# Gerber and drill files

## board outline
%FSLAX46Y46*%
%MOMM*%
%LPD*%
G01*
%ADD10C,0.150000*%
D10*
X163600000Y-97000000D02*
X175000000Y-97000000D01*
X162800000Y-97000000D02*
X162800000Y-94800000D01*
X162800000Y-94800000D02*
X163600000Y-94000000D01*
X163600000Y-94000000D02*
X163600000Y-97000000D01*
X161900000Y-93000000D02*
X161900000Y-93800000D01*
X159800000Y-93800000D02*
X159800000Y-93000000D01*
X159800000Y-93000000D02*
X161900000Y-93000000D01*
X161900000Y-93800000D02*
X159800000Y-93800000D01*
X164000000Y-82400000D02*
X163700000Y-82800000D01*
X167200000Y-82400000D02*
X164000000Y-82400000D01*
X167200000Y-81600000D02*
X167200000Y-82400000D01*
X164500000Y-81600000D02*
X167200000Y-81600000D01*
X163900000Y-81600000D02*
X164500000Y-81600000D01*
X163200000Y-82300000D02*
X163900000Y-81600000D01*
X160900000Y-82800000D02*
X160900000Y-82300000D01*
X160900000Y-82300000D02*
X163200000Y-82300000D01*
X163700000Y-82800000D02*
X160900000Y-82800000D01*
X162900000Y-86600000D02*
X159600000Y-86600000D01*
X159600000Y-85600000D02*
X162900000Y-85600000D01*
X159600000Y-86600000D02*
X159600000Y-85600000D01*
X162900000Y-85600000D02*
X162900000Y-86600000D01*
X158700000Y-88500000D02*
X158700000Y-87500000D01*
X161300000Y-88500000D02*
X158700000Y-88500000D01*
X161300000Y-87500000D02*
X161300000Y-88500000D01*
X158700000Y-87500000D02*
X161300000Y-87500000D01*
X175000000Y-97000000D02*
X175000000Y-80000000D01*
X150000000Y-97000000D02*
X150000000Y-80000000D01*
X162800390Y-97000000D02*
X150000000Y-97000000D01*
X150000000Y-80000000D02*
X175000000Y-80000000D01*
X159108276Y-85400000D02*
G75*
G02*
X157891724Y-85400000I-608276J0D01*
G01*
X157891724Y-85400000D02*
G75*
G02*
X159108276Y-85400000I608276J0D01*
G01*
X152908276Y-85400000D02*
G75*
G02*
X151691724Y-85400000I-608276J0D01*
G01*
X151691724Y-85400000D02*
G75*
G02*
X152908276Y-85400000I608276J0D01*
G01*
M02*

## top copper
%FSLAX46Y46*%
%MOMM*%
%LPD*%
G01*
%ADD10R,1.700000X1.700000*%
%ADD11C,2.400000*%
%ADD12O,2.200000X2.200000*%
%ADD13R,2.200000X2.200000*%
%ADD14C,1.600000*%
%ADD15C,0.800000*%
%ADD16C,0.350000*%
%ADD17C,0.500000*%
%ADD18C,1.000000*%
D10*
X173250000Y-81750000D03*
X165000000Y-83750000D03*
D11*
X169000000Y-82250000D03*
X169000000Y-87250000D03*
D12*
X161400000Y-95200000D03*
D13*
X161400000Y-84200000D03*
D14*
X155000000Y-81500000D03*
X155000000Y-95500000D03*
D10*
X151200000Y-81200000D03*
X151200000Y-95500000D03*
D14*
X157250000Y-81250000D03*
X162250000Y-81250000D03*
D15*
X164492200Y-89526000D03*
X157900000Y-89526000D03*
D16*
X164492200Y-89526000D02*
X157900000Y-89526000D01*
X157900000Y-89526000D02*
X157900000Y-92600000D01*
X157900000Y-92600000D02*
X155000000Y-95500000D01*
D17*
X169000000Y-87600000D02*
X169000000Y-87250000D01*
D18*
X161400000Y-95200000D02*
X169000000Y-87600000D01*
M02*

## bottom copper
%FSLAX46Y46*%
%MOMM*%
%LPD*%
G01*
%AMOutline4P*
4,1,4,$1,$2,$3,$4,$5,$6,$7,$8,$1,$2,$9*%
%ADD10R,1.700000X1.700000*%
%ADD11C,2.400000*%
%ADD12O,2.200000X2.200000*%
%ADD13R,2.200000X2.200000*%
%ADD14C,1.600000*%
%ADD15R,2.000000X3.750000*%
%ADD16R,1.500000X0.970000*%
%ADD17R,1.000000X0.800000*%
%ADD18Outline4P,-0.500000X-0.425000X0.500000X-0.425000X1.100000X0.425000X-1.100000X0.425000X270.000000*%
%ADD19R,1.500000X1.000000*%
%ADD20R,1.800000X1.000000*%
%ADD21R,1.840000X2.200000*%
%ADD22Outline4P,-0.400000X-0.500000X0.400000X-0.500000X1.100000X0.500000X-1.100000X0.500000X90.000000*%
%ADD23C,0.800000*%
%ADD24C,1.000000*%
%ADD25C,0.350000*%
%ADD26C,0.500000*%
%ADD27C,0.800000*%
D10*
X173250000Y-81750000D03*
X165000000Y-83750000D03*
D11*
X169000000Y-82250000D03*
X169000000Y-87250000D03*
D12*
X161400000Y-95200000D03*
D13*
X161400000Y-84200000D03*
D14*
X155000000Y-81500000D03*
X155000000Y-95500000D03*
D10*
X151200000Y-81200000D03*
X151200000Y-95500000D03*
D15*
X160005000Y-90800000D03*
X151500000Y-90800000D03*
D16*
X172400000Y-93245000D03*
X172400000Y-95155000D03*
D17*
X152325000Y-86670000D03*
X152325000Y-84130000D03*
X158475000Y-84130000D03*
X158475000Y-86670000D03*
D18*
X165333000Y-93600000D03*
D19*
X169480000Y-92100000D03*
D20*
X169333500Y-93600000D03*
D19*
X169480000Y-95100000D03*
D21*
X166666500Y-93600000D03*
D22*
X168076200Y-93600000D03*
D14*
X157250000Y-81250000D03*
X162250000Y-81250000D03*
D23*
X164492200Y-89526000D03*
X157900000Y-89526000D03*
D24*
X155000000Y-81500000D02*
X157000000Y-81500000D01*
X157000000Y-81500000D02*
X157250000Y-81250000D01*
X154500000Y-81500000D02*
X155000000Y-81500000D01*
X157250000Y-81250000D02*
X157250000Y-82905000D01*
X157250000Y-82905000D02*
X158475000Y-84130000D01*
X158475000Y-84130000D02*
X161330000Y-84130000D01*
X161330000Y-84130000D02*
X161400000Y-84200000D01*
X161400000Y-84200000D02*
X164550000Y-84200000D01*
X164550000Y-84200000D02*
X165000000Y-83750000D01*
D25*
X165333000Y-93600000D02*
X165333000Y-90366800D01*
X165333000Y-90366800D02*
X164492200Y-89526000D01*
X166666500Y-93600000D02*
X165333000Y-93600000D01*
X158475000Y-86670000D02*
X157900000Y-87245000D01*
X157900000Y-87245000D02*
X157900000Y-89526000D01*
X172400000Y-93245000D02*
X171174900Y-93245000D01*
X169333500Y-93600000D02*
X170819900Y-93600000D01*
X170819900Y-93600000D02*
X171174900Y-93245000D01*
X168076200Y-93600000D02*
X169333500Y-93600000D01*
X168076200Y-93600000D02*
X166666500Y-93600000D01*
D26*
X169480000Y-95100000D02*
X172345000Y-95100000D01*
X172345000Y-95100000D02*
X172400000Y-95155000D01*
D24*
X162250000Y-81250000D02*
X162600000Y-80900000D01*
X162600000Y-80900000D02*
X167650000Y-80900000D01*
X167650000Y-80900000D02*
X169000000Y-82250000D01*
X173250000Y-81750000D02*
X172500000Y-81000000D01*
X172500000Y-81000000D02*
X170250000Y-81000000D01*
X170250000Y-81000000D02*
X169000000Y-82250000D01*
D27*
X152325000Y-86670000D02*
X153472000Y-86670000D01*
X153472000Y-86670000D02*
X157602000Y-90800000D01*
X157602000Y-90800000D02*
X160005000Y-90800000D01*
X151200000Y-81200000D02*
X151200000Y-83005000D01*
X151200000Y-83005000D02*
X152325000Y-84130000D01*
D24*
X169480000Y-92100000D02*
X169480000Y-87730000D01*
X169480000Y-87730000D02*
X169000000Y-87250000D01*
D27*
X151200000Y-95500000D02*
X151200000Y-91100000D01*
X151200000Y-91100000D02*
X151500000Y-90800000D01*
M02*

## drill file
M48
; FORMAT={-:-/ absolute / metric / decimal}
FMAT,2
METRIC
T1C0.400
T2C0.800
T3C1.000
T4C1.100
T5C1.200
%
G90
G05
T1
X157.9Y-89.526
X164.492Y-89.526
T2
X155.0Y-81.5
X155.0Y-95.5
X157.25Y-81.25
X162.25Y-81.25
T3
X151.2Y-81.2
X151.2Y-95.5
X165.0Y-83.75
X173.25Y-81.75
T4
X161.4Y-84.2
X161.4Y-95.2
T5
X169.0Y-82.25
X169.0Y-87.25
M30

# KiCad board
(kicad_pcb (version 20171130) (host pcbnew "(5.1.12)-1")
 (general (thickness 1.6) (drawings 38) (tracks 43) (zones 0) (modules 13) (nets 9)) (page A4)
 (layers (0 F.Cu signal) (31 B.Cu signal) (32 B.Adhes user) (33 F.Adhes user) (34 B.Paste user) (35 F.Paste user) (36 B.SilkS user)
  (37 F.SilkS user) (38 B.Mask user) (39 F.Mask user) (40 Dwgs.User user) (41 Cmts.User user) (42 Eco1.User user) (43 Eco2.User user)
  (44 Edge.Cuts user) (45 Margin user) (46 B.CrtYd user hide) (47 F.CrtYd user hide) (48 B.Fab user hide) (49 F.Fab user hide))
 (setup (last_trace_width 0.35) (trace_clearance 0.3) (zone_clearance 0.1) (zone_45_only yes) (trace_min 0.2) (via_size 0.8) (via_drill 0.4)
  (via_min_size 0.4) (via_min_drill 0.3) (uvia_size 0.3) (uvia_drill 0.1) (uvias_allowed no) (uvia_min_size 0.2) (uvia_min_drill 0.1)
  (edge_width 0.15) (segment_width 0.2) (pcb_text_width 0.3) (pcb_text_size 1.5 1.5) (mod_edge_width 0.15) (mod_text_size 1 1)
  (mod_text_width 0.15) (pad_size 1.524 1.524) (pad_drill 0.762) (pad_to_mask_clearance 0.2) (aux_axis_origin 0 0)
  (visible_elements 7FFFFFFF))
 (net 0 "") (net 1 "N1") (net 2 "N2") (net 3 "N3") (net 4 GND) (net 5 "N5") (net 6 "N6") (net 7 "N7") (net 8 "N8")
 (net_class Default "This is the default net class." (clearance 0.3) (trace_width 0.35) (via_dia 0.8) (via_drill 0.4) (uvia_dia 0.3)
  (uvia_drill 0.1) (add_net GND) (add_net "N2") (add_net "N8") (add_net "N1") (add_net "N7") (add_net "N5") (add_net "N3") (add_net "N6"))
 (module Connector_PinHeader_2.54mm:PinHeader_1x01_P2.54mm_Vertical (layer F.Cu) (at 173.25 81.75)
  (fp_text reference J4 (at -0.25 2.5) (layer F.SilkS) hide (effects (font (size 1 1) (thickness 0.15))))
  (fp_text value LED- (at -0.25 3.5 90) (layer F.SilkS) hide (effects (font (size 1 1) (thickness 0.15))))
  (pad 1 thru_hole rect (at 0 0) (size 1.7 1.7) (drill 1) (layers *.Cu *.Mask) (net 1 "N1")))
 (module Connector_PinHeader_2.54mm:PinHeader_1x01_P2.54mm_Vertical (layer F.Cu) (at 165 83.75)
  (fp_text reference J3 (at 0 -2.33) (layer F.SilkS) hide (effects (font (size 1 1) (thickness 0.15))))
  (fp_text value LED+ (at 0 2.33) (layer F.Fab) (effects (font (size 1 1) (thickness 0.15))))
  (pad 1 thru_hole rect (at 0 0) (size 1.7 1.7) (drill 1) (layers *.Cu *.Mask) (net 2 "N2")))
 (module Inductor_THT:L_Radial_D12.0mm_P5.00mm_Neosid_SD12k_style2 (layer F.Cu) (at 169 82.25 270)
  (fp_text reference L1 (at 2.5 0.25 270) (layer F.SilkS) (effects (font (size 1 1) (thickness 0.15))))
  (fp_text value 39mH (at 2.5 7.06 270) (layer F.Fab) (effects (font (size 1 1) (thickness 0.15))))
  (pad 1 thru_hole circle (at 0 0 270) (size 2.4 2.4) (drill 1.2) (layers *.Cu *.Mask) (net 1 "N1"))
  (pad 2 thru_hole circle (at 5 0 270) (size 2.4 2.4) (drill 1.2) (layers *.Cu *.Mask) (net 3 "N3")))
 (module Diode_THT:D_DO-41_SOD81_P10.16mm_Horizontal (layer F.Cu) (at 161.4 84.2 270)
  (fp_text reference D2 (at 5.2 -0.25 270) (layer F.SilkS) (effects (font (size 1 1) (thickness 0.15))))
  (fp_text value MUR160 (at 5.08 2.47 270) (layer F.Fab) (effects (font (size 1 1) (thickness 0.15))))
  (pad 2 thru_hole oval (at 11 0 270) (size 2.2 2.2) (drill 1.1) (layers *.Cu *.Mask) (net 3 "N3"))
  (pad 1 thru_hole rect (at 0 0 270) (size 2.2 2.2) (drill 1.1) (layers *.Cu *.Mask) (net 2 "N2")))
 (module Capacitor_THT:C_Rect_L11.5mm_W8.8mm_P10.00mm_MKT (layer F.Cu) (at 155 83.5 270)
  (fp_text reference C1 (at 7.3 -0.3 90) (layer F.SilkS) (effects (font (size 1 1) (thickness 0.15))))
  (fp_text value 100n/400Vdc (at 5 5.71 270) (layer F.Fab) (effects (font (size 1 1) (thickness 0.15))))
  (pad 1 thru_hole circle (at -2 0 270) (size 1.6 1.6) (drill 0.8) (layers *.Cu *.Mask) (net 2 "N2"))
  (pad 2 thru_hole circle (at 12 0 270) (size 1.6 1.6) (drill 0.8) (layers *.Cu *.Mask) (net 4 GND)))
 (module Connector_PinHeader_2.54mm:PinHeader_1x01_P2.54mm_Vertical (layer F.Cu) (at 151.2 81.2)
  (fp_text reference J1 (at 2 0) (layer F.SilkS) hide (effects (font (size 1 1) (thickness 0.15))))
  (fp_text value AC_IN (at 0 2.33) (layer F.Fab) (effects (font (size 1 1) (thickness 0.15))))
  (pad 1 thru_hole rect (at 0 0) (size 1.7 1.7) (drill 1) (layers *.Cu *.Mask) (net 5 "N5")))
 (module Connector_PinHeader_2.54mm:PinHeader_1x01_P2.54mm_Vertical (layer F.Cu) (at 151.2 95.5)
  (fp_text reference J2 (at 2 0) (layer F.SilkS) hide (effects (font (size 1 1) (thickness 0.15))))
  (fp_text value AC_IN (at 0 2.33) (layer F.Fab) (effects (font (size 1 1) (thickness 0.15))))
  (pad 1 thru_hole rect (at 0 0) (size 1.7 1.7) (drill 1) (layers *.Cu *.Mask) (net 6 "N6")))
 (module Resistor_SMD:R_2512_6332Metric (layer B.Cu) (at 157 90.8 180)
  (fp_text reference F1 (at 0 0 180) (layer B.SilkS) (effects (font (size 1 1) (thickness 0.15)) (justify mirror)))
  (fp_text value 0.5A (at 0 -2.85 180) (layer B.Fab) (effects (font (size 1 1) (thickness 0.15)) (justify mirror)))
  (pad 1 smd rect (at -3.005 0 180) (size 2 3.75) (layers B.Cu B.Paste B.Mask) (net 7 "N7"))
  (pad 2 smd rect (at 5.5 0 180) (size 2 3.75) (layers B.Cu B.Paste B.Mask) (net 6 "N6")))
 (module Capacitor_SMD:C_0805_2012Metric (layer B.Cu) (at 172.4 94.2 270)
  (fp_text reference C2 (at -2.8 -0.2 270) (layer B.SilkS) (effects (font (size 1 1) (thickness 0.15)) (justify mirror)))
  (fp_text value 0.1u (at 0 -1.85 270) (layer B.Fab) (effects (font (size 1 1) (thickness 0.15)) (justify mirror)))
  (pad 1 smd rect (at -0.955 0 270) (size 0.97 1.5) (layers B.Cu B.Paste B.Mask) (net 4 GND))
  (pad 2 smd rect (at 0.955 0 270) (size 0.97 1.5) (layers B.Cu B.Paste B.Mask) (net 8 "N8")))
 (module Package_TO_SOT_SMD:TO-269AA (layer B.Cu) (at 155.4 85.4)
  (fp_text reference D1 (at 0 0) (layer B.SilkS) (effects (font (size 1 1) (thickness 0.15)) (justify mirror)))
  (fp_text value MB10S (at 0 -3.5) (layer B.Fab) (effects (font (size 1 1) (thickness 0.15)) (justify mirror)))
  (pad 1 smd rect (at -3.075 1.27) (size 1 0.8) (layers B.Cu B.Paste B.Mask) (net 7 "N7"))
  (pad 2 smd rect (at -3.075 -1.27) (size 1 0.8) (layers B.Cu B.Paste B.Mask) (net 5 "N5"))
  (pad 3 smd rect (at 3.075 -1.27) (size 1 0.8) (layers B.Cu B.Paste B.Mask) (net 2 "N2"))
  (pad 4 smd rect (at 3.075 1.27) (size 1 0.8) (layers B.Cu B.Paste B.Mask) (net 4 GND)))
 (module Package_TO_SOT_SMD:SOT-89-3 (layer B.Cu) (at 168 93.6 180)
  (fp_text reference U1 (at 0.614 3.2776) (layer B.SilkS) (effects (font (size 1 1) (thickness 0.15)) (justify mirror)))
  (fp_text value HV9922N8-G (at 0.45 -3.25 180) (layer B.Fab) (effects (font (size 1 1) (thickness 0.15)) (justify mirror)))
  (pad 2 smd trapezoid (at 2.667 0 270) (size 1.6 0.85) (rect_delta 0 -0.6) (layers B.Cu B.Paste B.Mask) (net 4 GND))
  (pad 1 smd rect (at -1.48 1.5 270) (size 1 1.5) (layers B.Cu B.Paste B.Mask) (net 3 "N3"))
  (pad 2 smd rect (at -1.3335 0 270) (size 1 1.8) (layers B.Cu B.Paste B.Mask) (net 4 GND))
  (pad 3 smd rect (at -1.48 -1.5 270) (size 1 1.5) (layers B.Cu B.Paste B.Mask) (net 8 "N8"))
  (pad 2 smd rect (at 1.3335 0 270) (size 2.2 1.84) (layers B.Cu B.Paste B.Mask) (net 4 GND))
  (pad 2 smd trapezoid (at -0.0762 0 90) (size 1.5 1) (rect_delta 0 -0.7) (layers B.Cu B.Paste B.Mask) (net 4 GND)))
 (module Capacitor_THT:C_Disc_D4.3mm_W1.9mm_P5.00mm (layer F.Cu) (at 157.25 81.25)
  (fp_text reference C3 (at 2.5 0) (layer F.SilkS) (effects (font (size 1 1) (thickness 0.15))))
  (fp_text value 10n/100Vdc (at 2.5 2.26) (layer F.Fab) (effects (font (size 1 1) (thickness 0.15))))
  (pad 1 thru_hole circle (at 0 0) (size 1.6 1.6) (drill 0.8) (layers *.Cu *.Mask) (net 2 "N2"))
  (pad 2 thru_hole circle (at 5 0) (size 1.6 1.6) (drill 0.8) (layers *.Cu *.Mask) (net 1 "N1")))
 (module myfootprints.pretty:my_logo (layer F.Cu) (at 170.942 93.98)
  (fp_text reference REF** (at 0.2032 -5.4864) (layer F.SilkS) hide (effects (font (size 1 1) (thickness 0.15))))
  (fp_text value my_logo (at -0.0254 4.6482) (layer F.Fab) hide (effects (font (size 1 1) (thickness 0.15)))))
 (gr_line (start 163.6 97) (end 175 97) (layer Edge.Cuts) (width 0.15))
 (gr_line (start 162.8 97) (end 162.8 94.8) (layer Edge.Cuts) (width 0.15))
 (gr_line (start 162.8 94.8) (end 163.6 94) (layer Edge.Cuts) (width 0.15))
 (gr_line (start 163.6 94) (end 163.6 97) (layer Edge.Cuts) (width 0.15))
 (gr_line (start 161.9 93) (end 161.9 93.8) (layer Edge.Cuts) (width 0.15))
 (gr_line (start 159.8 93.8) (end 159.8 93) (layer Edge.Cuts) (width 0.15))
 (gr_line (start 159.8 93) (end 161.9 93) (layer Edge.Cuts) (width 0.15))
 (gr_line (start 161.9 93.8) (end 159.8 93.8) (layer Edge.Cuts) (width 0.15))
 (gr_line (start 164 82.4) (end 163.7 82.8) (layer Edge.Cuts) (width 0.15))
 (gr_line (start 167.2 82.4) (end 164 82.4) (layer Edge.Cuts) (width 0.15))
 (gr_line (start 167.2 81.6) (end 167.2 82.4) (layer Edge.Cuts) (width 0.15))
 (gr_line (start 164.5 81.6) (end 167.2 81.6) (layer Edge.Cuts) (width 0.15))
 (gr_line (start 163.9 81.6) (end 164.5 81.6) (layer Edge.Cuts) (width 0.15))
 (gr_line (start 163.2 82.3) (end 163.9 81.6) (layer Edge.Cuts) (width 0.15))
 (gr_line (start 160.9 82.8) (end 160.9 82.3) (layer Edge.Cuts) (width 0.15))
 (gr_line (start 160.9 82.3) (end 163.2 82.3) (layer Edge.Cuts) (width 0.15))
 (gr_line (start 163.7 82.8) (end 160.9 82.8) (layer Edge.Cuts) (width 0.15))
 (gr_line (start 162.9 86.6) (end 159.6 86.6) (layer Edge.Cuts) (width 0.15))
 (gr_line (start 159.6 85.6) (end 162.9 85.6) (layer Edge.Cuts) (width 0.15))
 (gr_line (start 159.6 86.6) (end 159.6 85.6) (layer Edge.Cuts) (width 0.15))
 (gr_line (start 162.9 85.6) (end 162.9 86.6) (layer Edge.Cuts) (width 0.15))
 (gr_line (start 158.7 88.5) (end 158.7 87.5) (layer Edge.Cuts) (width 0.15))
 (gr_line (start 161.3 88.5) (end 158.7 88.5) (layer Edge.Cuts) (width 0.15))
 (gr_line (start 161.3 87.5) (end 161.3 88.5) (layer Edge.Cuts) (width 0.15))
 (gr_line (start 158.7 87.5) (end 161.3 87.5) (layer Edge.Cuts) (width 0.15))
 (gr_line (start 175 97) (end 175 80) (layer Edge.Cuts) (width 0.15))
 (gr_line (start 150 97) (end 150 80) (layer Edge.Cuts) (width 0.15))
 (gr_line (start 162.80039 97) (end 150 97) (layer Edge.Cuts) (width 0.15))
 (gr_line (start 150 80) (end 175 80) (layer Edge.Cuts) (width 0.15))
 (gr_circle (center 158.5 85.4) (end 159.108276 85.4) (layer Edge.Cuts) (width 0.15))
 (gr_circle (center 152.3 85.4) (end 152.908276 85.4) (layer Edge.Cuts) (width 0.15))
 (segment (start 155 81.5) (end 157 81.5) (width 1) (layer B.Cu) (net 2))
 (segment (start 157 81.5) (end 157.25 81.25) (width 1) (layer B.Cu) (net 2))
 (segment (start 154.5 81.5) (end 155 81.5) (width 1) (layer B.Cu) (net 2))
 (segment (start 157.25 81.25) (end 157.25 82.905) (width 1) (layer B.Cu) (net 2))
 (segment (start 157.25 82.905) (end 158.475 84.13) (width 1) (layer B.Cu) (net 2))
 (segment (start 158.475 84.13) (end 161.33 84.13) (width 1) (layer B.Cu) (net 2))
 (segment (start 161.33 84.13) (end 161.4 84.2) (width 1) (layer B.Cu) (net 2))
 (segment (start 161.4 84.2) (end 164.55 84.2) (width 1) (layer B.Cu) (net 2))
 (segment (start 164.55 84.2) (end 165 83.75) (width 1) (layer B.Cu) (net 2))
 (segment (start 165.333 93.6) (end 165.333 90.3668) (width 0.35) (layer B.Cu) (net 4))
 (segment (start 165.333 90.3668) (end 164.4922 89.526) (width 0.35) (layer B.Cu) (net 4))
 (segment (start 164.4922 89.526) (end 157.9 89.526) (width 0.35) (layer F.Cu) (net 4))
 (segment (start 166.6665 93.6) (end 165.333 93.6) (width 0.35) (layer B.Cu) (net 4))
 (segment (start 157.9 89.526) (end 157.9 92.6) (width 0.35) (layer F.Cu) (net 4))
 (segment (start 157.9 92.6) (end 155 95.5) (width 0.35) (layer F.Cu) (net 4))
 (segment (start 158.475 86.67) (end 157.9 87.245) (width 0.35) (layer B.Cu) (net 4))
 (segment (start 157.9 87.245) (end 157.9 89.526) (width 0.35) (layer B.Cu) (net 4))
 (segment (start 172.4 93.245) (end 171.1749 93.245) (width 0.35) (layer B.Cu) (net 4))
 (segment (start 169.3335 93.6) (end 170.8199 93.6) (width 0.35) (layer B.Cu) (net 4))
 (segment (start 170.8199 93.6) (end 171.1749 93.245) (width 0.35) (layer B.Cu) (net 4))
 (segment (start 168.0762 93.6) (end 169.3335 93.6) (width 0.35) (layer B.Cu) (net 4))
 (segment (start 168.0762 93.6) (end 166.6665 93.6) (width 0.35) (layer B.Cu) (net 4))
 (via (at 164.4922 89.526) (size 0.8) (layers F.Cu B.Cu) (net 4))
 (via (at 157.9 89.526) (size 0.8) (layers F.Cu B.Cu) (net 4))
 (segment (start 169.48 95.1) (end 172.345 95.1) (width 0.5) (layer B.Cu) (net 8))
 (segment (start 172.345 95.1) (end 172.4 95.155) (width 0.5) (layer B.Cu) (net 8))
 (segment (start 162.25 81.25) (end 162.6 80.9) (width 1) (layer B.Cu) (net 1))
 (segment (start 162.6 80.9) (end 167.65 80.9) (width 1) (layer B.Cu) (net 1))
 (segment (start 167.65 80.9) (end 169 82.25) (width 1) (layer B.Cu) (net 1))
 (segment (start 173.25 81.75) (end 172.5 81) (width 1) (layer B.Cu) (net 1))
 (segment (start 172.5 81) (end 170.25 81) (width 1) (layer B.Cu) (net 1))
 (segment (start 170.25 81) (end 169 82.25) (width 1) (layer B.Cu) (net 1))
 (segment (start 152.325 86.67) (end 153.472 86.67) (width 0.8) (layer B.Cu) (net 7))
 (segment (start 153.472 86.67) (end 157.602 90.8) (width 0.8) (layer B.Cu) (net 7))
 (segment (start 157.602 90.8) (end 160.005 90.8) (width 0.8) (layer B.Cu) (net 7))
 (segment (start 151.2 81.2) (end 151.2 83.005) (width 0.8) (layer B.Cu) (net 5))
 (segment (start 151.2 83.005) (end 152.325 84.13) (width 0.8) (layer B.Cu) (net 5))
 (segment (start 169 87.6) (end 169 87.25) (width 0.5) (layer F.Cu) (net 3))
 (segment (start 161.4 95.2) (end 169 87.6) (width 1) (layer F.Cu) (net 3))
 (segment (start 169.48 92.1) (end 169.48 87.73) (width 1) (layer B.Cu) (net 3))
 (segment (start 169.48 87.73) (end 169 87.25) (width 1) (layer B.Cu) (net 3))
 (segment (start 151.2 95.5) (end 151.2 91.1) (width 0.8) (layer B.Cu) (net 6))
 (segment (start 151.2 91.1) (end 151.5 90.8) (width 0.8) (layer B.Cu) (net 6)))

